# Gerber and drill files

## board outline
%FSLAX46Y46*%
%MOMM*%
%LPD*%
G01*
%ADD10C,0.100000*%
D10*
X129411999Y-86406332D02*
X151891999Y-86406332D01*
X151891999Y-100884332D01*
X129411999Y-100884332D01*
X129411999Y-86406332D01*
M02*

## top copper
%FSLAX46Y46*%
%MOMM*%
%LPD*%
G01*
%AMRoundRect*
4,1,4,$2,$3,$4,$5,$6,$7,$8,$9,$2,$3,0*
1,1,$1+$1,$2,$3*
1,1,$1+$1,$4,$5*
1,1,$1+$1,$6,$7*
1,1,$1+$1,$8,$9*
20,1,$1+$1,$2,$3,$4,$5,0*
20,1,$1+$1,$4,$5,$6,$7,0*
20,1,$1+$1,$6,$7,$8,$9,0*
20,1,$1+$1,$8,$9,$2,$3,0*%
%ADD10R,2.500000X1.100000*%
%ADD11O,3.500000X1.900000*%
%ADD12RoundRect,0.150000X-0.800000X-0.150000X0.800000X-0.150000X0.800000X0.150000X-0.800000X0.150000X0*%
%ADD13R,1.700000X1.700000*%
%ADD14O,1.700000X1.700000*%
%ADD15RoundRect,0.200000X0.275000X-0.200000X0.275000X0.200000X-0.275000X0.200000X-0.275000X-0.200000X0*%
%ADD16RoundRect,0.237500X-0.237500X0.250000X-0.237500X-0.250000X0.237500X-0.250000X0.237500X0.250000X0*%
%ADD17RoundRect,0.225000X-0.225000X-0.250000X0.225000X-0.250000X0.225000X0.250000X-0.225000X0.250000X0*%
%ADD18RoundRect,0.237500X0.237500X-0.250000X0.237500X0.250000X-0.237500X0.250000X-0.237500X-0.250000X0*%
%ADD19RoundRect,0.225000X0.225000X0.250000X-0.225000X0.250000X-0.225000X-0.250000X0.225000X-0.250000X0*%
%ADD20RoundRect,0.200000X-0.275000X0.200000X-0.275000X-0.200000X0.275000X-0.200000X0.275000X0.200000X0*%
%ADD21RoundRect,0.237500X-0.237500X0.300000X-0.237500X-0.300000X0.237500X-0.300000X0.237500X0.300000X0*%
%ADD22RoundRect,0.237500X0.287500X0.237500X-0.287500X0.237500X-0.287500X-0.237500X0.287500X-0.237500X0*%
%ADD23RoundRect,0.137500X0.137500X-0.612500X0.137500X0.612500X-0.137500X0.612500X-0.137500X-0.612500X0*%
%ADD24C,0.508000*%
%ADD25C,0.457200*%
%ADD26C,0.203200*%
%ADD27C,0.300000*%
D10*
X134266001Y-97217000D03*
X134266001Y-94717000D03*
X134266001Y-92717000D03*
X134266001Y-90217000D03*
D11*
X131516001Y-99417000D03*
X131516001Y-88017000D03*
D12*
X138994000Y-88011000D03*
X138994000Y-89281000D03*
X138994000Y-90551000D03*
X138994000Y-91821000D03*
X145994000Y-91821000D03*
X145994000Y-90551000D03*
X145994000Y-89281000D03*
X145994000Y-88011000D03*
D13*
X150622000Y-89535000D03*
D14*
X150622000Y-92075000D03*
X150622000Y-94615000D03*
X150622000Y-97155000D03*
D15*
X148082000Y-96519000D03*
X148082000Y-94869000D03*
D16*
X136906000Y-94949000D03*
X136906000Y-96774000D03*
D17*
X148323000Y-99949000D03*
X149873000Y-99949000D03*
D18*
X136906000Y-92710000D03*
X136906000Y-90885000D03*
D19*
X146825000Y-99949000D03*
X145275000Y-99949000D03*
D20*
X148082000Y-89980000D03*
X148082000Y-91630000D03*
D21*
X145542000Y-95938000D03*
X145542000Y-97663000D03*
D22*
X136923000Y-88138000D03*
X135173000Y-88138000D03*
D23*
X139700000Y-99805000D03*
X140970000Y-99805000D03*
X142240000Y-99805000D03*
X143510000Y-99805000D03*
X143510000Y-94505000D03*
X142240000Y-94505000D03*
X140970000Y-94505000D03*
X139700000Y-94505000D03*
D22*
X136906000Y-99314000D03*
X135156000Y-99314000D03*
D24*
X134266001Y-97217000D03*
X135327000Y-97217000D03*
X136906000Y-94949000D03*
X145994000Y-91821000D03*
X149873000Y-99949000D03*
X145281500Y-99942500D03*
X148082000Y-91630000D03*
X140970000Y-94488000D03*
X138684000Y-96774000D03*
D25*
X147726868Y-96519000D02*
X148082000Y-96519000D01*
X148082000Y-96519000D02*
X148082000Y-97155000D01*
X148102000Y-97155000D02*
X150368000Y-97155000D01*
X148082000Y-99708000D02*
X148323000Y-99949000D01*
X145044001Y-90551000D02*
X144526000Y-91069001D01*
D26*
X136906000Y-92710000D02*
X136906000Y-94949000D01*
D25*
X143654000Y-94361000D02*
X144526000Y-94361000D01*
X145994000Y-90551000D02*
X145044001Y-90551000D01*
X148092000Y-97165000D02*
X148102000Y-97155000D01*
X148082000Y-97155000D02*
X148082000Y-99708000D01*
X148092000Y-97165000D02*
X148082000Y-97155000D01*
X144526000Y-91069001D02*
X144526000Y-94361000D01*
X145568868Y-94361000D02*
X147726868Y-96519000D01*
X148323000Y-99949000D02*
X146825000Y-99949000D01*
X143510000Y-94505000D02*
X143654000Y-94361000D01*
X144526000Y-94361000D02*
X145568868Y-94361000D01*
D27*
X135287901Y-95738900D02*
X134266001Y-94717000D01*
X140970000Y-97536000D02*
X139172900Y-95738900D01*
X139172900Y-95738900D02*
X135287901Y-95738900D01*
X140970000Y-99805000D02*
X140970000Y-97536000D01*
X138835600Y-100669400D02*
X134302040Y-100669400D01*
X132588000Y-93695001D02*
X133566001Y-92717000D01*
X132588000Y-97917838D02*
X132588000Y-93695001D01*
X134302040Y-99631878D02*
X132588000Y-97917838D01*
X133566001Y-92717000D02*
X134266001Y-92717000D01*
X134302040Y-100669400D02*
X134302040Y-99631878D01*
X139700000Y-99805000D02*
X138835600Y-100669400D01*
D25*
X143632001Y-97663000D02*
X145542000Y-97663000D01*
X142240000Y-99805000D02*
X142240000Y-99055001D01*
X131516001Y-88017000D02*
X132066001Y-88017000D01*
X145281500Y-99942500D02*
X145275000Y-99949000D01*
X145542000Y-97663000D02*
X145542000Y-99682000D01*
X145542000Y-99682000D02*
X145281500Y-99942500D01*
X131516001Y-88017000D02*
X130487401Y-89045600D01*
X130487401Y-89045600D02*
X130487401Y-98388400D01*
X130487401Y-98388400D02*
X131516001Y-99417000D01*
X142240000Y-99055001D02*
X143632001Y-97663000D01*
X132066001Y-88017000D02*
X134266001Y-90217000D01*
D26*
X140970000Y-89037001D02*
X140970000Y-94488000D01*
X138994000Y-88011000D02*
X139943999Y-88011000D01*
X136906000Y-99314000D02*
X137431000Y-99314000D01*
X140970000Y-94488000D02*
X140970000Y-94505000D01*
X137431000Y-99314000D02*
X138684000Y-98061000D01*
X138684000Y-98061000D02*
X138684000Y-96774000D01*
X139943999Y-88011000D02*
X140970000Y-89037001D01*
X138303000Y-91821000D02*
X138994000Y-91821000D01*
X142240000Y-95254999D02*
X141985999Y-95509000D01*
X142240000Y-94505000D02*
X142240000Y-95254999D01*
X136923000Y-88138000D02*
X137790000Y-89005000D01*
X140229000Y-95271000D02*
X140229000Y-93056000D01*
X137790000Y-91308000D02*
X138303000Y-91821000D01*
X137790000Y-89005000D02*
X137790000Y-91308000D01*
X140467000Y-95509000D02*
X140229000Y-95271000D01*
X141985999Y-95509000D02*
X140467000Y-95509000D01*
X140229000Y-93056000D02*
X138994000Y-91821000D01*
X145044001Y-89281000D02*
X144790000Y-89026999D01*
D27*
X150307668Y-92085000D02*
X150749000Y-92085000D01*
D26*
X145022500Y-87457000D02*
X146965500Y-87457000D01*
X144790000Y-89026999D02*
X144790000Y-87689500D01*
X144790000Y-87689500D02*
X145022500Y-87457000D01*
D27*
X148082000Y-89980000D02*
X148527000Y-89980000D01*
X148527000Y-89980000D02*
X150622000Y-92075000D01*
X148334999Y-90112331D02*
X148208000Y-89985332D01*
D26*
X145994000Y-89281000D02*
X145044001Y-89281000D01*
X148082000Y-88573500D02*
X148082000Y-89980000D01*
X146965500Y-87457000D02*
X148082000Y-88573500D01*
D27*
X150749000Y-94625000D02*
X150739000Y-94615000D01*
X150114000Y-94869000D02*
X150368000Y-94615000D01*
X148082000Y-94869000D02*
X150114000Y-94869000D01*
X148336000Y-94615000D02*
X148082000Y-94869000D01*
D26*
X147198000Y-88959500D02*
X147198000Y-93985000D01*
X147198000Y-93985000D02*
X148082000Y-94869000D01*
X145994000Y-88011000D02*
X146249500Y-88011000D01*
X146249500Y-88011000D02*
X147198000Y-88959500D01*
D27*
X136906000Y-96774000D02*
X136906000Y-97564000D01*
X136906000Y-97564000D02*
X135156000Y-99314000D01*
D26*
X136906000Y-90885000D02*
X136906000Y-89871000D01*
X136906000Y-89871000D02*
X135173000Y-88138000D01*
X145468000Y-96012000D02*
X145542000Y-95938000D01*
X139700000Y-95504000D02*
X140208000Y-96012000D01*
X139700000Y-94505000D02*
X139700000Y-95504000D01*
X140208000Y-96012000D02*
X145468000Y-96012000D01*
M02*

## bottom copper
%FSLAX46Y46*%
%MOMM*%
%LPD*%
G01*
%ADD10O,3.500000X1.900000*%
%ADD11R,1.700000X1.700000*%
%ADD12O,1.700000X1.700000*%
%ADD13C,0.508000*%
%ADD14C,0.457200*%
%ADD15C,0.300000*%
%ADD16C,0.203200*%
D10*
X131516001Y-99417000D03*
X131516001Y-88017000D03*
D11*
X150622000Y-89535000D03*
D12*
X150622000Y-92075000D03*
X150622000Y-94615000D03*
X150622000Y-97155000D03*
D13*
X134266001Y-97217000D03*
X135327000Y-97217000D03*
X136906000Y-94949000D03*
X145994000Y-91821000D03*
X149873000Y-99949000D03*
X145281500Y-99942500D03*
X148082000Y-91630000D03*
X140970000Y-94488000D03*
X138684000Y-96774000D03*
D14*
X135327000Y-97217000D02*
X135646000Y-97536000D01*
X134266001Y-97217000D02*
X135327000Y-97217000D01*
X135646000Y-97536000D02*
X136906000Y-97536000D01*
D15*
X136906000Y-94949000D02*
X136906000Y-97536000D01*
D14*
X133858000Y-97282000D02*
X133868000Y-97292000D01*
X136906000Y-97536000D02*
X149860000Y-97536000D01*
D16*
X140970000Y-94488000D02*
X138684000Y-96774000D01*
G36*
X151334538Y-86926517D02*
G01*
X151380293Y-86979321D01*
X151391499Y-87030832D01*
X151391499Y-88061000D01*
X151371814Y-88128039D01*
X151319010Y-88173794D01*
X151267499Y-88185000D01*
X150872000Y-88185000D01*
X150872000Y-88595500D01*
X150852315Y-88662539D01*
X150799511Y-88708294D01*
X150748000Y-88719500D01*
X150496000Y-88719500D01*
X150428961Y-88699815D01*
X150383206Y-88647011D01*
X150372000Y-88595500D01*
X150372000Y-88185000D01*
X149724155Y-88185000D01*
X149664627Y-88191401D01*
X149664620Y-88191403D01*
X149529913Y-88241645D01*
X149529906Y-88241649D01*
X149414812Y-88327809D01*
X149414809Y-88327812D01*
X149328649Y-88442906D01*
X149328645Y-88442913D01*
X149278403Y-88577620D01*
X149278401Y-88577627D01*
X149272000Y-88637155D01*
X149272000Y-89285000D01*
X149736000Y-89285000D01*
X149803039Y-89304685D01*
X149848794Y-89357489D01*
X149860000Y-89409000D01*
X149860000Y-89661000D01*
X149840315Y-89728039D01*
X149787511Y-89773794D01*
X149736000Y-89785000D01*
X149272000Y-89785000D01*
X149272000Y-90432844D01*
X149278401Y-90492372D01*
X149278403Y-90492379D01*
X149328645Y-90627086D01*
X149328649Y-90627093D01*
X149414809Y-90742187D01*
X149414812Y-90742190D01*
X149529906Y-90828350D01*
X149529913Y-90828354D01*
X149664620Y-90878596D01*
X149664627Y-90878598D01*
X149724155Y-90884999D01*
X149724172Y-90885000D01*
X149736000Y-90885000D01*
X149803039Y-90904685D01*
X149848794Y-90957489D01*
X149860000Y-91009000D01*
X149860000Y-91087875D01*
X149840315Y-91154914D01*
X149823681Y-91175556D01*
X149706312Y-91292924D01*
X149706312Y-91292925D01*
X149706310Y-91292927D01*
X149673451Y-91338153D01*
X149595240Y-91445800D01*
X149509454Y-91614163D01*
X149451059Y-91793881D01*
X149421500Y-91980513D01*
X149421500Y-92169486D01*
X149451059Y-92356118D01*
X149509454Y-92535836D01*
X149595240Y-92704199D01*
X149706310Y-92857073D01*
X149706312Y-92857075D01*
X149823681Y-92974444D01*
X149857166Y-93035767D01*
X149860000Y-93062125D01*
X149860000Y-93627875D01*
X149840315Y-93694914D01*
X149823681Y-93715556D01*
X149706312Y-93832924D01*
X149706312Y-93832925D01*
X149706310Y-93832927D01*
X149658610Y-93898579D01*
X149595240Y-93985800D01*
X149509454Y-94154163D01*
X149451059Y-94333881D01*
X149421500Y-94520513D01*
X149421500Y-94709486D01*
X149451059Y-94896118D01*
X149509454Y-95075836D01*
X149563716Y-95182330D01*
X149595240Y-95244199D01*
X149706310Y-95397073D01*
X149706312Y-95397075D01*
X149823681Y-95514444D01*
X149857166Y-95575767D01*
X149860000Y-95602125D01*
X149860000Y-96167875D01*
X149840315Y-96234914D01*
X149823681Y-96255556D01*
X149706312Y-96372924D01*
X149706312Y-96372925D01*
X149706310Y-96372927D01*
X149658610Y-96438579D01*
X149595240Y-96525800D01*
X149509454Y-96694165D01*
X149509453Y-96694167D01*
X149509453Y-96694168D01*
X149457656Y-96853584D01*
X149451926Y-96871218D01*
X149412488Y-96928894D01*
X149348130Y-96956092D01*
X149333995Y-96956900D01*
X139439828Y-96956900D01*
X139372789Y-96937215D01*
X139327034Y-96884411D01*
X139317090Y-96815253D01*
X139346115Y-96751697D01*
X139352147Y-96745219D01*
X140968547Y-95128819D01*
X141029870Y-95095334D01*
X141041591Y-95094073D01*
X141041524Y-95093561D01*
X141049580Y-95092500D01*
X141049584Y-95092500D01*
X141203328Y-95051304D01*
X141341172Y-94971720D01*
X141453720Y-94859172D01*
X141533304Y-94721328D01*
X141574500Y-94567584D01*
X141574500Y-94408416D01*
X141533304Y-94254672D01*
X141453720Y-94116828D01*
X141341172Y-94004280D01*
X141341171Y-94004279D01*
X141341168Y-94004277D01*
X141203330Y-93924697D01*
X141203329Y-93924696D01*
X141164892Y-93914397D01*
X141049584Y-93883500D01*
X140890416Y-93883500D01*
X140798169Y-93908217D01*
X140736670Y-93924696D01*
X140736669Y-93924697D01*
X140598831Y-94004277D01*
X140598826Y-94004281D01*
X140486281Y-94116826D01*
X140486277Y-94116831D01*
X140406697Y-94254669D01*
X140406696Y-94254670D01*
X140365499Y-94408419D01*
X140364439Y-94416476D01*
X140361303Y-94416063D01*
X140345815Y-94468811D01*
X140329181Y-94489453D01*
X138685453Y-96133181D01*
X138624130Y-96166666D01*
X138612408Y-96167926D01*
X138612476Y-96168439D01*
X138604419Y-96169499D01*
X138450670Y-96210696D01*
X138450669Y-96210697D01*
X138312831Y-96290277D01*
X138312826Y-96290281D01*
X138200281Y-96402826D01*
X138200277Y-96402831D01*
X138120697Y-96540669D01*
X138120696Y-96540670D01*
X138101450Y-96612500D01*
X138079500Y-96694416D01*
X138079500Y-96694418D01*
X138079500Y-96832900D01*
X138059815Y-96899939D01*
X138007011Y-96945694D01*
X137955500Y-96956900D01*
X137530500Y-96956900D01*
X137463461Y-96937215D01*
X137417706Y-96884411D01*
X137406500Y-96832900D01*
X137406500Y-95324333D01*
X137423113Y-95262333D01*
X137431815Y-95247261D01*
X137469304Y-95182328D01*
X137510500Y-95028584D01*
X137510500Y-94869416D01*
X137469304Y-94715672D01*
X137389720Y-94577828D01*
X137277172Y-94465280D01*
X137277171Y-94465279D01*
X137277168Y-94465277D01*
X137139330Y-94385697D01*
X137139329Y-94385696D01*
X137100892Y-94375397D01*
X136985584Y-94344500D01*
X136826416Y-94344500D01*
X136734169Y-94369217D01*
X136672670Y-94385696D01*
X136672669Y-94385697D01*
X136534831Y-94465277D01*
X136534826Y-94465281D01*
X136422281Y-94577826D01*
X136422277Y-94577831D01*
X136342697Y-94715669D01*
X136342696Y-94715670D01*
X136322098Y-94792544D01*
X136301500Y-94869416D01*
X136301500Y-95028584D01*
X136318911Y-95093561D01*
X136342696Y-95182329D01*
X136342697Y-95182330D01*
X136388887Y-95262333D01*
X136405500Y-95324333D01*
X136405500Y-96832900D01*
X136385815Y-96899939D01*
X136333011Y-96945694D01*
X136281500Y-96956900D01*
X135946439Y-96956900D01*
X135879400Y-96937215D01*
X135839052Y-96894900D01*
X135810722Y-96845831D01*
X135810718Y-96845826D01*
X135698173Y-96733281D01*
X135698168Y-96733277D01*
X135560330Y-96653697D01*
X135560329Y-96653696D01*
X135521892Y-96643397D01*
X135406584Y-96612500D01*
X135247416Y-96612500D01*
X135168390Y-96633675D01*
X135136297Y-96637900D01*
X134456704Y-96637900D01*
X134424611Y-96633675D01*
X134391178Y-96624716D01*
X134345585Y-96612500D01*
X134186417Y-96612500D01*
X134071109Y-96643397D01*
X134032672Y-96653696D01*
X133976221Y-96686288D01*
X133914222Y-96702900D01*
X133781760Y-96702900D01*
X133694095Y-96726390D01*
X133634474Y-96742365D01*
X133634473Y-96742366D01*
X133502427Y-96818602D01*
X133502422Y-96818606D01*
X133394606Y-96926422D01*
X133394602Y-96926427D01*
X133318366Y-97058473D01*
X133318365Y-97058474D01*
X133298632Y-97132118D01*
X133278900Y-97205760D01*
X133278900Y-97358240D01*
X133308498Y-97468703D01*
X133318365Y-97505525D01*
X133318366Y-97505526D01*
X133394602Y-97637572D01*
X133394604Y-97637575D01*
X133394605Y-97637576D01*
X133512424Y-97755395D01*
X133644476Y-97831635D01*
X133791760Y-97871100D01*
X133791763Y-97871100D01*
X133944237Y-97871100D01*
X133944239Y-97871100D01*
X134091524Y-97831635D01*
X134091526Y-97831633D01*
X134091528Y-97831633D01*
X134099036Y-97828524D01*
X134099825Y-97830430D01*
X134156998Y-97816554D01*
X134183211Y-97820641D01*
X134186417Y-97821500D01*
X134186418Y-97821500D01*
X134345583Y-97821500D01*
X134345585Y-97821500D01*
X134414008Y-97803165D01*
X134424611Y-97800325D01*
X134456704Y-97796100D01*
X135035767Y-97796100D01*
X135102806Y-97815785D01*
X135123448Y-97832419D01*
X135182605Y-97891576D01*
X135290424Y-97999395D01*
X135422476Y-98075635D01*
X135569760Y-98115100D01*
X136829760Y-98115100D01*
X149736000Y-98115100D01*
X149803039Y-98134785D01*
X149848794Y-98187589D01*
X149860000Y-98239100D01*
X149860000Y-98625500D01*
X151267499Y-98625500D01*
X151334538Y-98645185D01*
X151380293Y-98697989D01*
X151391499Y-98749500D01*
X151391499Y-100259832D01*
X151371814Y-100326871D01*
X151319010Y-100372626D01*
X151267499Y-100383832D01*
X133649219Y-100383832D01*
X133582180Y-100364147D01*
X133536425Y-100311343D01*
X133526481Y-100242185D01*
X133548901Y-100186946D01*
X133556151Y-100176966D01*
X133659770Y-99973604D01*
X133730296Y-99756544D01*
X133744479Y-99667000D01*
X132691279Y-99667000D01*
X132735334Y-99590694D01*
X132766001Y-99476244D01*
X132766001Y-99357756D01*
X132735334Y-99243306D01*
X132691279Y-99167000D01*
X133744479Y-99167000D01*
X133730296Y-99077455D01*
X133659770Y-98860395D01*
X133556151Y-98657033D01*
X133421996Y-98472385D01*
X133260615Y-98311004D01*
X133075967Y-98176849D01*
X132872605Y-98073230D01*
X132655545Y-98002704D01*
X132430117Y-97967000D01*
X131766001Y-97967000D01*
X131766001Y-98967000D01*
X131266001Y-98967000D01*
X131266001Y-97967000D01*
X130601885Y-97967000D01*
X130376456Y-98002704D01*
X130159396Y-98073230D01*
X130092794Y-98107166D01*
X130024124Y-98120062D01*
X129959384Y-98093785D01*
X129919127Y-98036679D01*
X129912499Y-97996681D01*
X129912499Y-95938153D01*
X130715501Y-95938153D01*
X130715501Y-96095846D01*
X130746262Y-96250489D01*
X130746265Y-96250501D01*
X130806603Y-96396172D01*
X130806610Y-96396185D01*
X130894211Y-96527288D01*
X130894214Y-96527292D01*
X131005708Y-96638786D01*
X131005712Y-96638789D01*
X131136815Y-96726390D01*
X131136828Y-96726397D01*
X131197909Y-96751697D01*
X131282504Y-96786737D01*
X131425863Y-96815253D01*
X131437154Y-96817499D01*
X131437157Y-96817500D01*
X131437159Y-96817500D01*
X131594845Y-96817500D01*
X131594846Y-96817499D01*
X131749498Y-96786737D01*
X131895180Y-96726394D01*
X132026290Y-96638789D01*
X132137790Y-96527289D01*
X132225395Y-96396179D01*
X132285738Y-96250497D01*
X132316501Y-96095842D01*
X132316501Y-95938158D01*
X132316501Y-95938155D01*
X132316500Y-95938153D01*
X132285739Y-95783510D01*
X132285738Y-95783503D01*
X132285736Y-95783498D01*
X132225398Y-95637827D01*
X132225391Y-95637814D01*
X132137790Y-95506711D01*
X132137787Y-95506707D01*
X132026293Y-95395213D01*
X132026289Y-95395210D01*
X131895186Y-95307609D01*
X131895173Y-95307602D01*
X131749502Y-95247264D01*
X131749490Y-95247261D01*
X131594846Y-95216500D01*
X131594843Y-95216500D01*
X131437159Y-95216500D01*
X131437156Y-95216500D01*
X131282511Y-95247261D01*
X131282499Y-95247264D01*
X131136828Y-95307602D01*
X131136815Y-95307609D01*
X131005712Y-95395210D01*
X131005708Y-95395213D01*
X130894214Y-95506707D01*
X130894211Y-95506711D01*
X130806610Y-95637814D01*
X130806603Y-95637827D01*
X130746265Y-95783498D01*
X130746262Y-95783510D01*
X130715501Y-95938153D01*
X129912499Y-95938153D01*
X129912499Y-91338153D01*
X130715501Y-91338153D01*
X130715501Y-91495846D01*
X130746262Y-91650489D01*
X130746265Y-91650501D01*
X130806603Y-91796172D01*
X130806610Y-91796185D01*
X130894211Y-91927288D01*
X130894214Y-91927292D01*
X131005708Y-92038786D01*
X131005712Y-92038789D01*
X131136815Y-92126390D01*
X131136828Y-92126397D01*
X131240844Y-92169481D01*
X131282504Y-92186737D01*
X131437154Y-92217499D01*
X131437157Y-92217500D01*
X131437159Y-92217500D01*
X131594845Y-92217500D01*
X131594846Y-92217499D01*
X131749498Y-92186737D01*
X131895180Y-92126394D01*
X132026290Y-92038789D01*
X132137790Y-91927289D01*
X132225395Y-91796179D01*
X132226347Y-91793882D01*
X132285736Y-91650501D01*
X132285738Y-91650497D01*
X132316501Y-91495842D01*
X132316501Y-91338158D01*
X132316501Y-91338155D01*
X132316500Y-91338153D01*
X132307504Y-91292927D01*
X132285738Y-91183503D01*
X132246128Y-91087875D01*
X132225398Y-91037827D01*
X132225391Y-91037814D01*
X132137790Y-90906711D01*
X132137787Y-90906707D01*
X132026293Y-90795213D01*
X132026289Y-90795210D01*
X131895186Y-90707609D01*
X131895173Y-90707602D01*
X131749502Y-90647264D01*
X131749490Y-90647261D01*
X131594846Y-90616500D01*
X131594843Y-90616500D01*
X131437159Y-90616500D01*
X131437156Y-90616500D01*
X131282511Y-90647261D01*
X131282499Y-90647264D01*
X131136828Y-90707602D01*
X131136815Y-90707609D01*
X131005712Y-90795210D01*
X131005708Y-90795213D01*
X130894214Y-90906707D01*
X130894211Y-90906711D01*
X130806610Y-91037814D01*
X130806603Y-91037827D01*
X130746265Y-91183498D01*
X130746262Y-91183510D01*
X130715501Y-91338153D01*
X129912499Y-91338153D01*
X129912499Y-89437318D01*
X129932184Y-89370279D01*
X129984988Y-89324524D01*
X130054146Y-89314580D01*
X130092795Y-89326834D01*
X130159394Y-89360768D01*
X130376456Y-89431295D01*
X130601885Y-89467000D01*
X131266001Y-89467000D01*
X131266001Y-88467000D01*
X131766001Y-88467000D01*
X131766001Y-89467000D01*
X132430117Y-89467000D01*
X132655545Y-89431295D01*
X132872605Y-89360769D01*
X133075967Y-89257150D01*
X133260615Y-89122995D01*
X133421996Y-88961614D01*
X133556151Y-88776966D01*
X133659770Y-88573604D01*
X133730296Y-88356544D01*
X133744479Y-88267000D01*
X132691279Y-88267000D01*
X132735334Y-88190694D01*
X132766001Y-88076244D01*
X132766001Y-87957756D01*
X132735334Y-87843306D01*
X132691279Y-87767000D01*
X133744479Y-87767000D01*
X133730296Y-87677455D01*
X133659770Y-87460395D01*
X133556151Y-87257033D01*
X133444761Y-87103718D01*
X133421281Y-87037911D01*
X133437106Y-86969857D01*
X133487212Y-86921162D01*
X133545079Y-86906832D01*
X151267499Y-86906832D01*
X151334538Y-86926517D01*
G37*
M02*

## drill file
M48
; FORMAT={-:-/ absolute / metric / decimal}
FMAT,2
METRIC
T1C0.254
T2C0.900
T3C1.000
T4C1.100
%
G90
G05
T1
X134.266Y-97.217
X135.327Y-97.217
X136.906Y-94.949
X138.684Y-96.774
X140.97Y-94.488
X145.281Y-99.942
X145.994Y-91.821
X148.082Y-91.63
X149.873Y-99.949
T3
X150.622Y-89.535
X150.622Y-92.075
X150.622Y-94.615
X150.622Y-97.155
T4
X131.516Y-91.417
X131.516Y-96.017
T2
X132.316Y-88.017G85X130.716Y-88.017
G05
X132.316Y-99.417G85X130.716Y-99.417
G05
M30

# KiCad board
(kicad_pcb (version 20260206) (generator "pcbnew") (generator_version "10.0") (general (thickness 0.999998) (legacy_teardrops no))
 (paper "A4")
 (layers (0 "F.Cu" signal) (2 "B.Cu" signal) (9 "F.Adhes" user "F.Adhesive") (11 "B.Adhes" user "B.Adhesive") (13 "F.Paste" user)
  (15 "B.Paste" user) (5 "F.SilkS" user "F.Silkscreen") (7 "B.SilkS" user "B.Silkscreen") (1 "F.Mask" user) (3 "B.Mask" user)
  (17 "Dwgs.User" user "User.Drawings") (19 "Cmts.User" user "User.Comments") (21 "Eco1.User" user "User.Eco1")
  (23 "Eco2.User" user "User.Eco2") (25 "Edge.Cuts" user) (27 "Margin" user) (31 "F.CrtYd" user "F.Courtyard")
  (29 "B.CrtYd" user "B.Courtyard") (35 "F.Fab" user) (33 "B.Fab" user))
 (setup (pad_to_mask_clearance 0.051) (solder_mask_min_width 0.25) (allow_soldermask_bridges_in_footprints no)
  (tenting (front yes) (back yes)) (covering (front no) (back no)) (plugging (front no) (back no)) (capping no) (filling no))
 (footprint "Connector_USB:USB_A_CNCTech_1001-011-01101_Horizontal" (layer "F.Cu") (at 124.616001 93.717 180)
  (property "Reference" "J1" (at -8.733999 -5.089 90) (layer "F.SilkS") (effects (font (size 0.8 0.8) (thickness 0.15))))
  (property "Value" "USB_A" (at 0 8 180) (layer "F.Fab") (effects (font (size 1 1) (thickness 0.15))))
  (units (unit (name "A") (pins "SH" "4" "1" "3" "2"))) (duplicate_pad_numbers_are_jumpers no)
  (pad "" np_thru_hole circle (at -6.9 -2.3 180) (size 1.1 1.1) (drill 1.1) (layers "*.Cu" "*.Mask"))
  (pad "" np_thru_hole circle (at -6.9 2.3 180) (size 1.1 1.1) (drill 1.1) (layers "*.Cu" "*.Mask"))
  (pad "1" smd rect (at -9.65 -3.5 180) (size 2.5 1.1) (layers "F.Cu" "F.Mask" "F.Paste") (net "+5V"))
  (pad "2" smd rect (at -9.65 -1 180) (size 2.5 1.1) (layers "F.Cu" "F.Mask" "F.Paste") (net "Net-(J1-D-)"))
  (pad "3" smd rect (at -9.65 1 180) (size 2.5 1.1) (layers "F.Cu" "F.Mask" "F.Paste") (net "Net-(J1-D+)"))
  (pad "4" smd rect (at -9.65 3.5 180) (size 2.5 1.1) (layers "F.Cu" "F.Mask" "F.Paste") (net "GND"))
  (pad "SH" thru_hole oval (at -6.9 -5.7 180) (size 3.5 1.9) (drill oval 2.5 0.9) (layers "*.Cu" "*.Mask") (remove_unused_layers no)
   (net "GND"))
  (pad "SH" thru_hole oval (at -6.9 5.7 180) (size 3.5 1.9) (drill oval 2.5 0.9) (layers "*.Cu" "*.Mask") (remove_unused_layers no)
   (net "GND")))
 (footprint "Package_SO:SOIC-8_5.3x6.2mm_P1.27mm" (layer "F.Cu") (at 142.494 89.916)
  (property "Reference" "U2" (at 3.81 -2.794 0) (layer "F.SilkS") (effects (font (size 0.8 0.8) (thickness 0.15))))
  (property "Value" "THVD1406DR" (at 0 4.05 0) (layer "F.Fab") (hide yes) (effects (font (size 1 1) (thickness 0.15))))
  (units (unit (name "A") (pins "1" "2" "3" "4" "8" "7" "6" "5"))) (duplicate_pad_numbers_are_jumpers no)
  (pad "1" smd roundrect (at -3.5 -1.905) (size 1.9 0.6) (layers "F.Cu" "F.Mask" "F.Paste") (roundrect_rratio 0.25) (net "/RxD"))
  (pad "2" smd roundrect (at -3.5 -0.635) (size 1.9 0.6) (layers "F.Cu" "F.Mask" "F.Paste") (roundrect_rratio 0.25)
   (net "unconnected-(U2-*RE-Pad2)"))
  (pad "3" smd roundrect (at -3.5 0.635) (size 1.9 0.6) (layers "F.Cu" "F.Mask" "F.Paste") (roundrect_rratio 0.25)
   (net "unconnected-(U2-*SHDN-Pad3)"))
  (pad "4" smd roundrect (at -3.5 1.905) (size 1.9 0.6) (layers "F.Cu" "F.Mask" "F.Paste") (roundrect_rratio 0.25) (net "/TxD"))
  (pad "5" smd roundrect (at 3.5 1.905) (size 1.9 0.6) (layers "F.Cu" "F.Mask" "F.Paste") (roundrect_rratio 0.25) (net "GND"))
  (pad "6" smd roundrect (at 3.5 0.635) (size 1.9 0.6) (layers "F.Cu" "F.Mask" "F.Paste") (roundrect_rratio 0.25) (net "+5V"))
  (pad "7" smd roundrect (at 3.5 -0.635) (size 1.9 0.6) (layers "F.Cu" "F.Mask" "F.Paste") (roundrect_rratio 0.25) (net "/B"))
  (pad "8" smd roundrect (at 3.5 -1.905) (size 1.9 0.6) (layers "F.Cu" "F.Mask" "F.Paste") (roundrect_rratio 0.25) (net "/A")))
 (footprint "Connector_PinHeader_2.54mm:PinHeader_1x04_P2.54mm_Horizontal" (layer "F.Cu") (at 150.622 89.535)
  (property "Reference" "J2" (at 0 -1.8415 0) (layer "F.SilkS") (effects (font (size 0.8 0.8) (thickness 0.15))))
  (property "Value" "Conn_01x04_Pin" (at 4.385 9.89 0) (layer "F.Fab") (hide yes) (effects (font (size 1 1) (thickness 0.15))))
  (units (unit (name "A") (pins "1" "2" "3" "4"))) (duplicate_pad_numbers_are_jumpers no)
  (pad "1" thru_hole rect (at 0 0) (size 1.7 1.7) (drill 1) (layers "*.Cu" "*.Mask") (remove_unused_layers no) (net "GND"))
  (pad "2" thru_hole oval (at 0 2.54) (size 1.7 1.7) (drill 1) (layers "*.Cu" "*.Mask") (remove_unused_layers no) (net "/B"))
  (pad "3" thru_hole oval (at 0 5.08) (size 1.7 1.7) (drill 1) (layers "*.Cu" "*.Mask") (remove_unused_layers no) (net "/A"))
  (pad "4" thru_hole oval (at 0 7.62) (size 1.7 1.7) (drill 1) (layers "*.Cu" "*.Mask") (remove_unused_layers no) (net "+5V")))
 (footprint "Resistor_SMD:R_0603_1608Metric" (layer "F.Cu") (at 148.082 95.694 90)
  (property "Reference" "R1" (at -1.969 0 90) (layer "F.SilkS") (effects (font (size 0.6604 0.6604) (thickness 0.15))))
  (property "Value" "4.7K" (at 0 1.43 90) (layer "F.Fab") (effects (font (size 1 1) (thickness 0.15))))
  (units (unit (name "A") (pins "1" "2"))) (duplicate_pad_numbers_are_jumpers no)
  (pad "1" smd roundrect (at -0.825 0 90) (size 0.8 0.95) (layers "F.Cu" "F.Mask" "F.Paste") (roundrect_rratio 0.25) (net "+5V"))
  (pad "2" smd roundrect (at 0.825 0 90) (size 0.8 0.95) (layers "F.Cu" "F.Mask" "F.Paste") (roundrect_rratio 0.25) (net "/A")))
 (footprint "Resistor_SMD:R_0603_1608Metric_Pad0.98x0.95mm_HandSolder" (layer "F.Cu") (at 136.906 95.8615 -90)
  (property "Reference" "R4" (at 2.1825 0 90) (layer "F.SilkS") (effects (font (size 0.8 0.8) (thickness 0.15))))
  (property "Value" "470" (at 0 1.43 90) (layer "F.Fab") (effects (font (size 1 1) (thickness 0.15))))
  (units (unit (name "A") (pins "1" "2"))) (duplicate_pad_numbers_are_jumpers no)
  (pad "1" smd roundrect (at -0.9125 0 270) (size 0.975 0.95) (layers "F.Cu" "F.Mask" "F.Paste") (roundrect_rratio 0.25) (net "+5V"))
  (pad "2" smd roundrect (at 0.9125 0 270) (size 0.975 0.95) (layers "F.Cu" "F.Mask" "F.Paste") (roundrect_rratio 0.25) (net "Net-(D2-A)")))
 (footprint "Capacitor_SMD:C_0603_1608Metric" (layer "F.Cu") (at 149.098 99.949)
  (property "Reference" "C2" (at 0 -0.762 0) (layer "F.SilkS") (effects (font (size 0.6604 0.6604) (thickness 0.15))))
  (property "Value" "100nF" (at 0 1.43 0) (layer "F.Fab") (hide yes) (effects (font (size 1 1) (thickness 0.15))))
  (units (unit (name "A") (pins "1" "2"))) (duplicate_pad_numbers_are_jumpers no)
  (pad "1" smd roundrect (at -0.775 0) (size 0.9 0.95) (layers "F.Cu" "F.Mask" "F.Paste") (roundrect_rratio 0.25) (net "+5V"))
  (pad "2" smd roundrect (at 0.775 0) (size 0.9 0.95) (layers "F.Cu" "F.Mask" "F.Paste") (roundrect_rratio 0.25) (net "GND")))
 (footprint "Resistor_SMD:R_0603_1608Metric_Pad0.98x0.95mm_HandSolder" (layer "F.Cu") (at 136.906 91.7975 90)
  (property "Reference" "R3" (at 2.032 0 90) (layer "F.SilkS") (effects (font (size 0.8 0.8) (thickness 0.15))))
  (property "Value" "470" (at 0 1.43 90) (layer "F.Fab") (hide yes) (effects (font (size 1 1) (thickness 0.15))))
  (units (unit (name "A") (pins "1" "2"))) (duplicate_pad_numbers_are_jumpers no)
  (pad "1" smd roundrect (at -0.9125 0 90) (size 0.975 0.95) (layers "F.Cu" "F.Mask" "F.Paste") (roundrect_rratio 0.25) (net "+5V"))
  (pad "2" smd roundrect (at 0.9125 0 90) (size 0.975 0.95) (layers "F.Cu" "F.Mask" "F.Paste") (roundrect_rratio 0.25) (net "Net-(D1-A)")))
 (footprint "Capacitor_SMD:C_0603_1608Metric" (layer "F.Cu") (at 146.05 99.949 180)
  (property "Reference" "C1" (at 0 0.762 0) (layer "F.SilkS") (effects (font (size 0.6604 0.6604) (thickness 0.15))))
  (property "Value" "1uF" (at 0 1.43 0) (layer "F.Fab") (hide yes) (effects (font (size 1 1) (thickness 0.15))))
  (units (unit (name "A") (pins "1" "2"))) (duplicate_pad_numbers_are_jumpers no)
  (pad "1" smd roundrect (at -0.775 0 180) (size 0.9 0.95) (layers "F.Cu" "F.Mask" "F.Paste") (roundrect_rratio 0.25) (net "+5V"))
  (pad "2" smd roundrect (at 0.775 0 180) (size 0.9 0.95) (layers "F.Cu" "F.Mask" "F.Paste") (roundrect_rratio 0.25) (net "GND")))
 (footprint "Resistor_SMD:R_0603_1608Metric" (layer "F.Cu") (at 148.082 90.805 -90)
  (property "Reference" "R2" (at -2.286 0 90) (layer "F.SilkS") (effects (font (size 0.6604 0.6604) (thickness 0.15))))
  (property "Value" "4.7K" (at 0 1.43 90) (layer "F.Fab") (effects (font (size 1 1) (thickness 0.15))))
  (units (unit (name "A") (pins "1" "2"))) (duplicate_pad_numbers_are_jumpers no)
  (pad "1" smd roundrect (at -0.825 0 270) (size 0.8 0.95) (layers "F.Cu" "F.Mask" "F.Paste") (roundrect_rratio 0.25) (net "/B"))
  (pad "2" smd roundrect (at 0.825 0 270) (size 0.8 0.95) (layers "F.Cu" "F.Mask" "F.Paste") (roundrect_rratio 0.25) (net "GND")))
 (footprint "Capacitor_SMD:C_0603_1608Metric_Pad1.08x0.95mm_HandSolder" (layer "F.Cu") (at 145.542 96.8005 -90)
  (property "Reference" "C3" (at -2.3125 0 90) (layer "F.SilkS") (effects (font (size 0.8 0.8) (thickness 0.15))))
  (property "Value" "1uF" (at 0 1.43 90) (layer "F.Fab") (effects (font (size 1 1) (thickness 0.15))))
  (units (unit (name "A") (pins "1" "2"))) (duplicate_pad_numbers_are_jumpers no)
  (pad "1" smd roundrect (at -0.8625 0 270) (size 1.075 0.95) (layers "F.Cu" "F.Mask" "F.Paste") (roundrect_rratio 0.25) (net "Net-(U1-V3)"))
  (pad "2" smd roundrect (at 0.8625 0 270) (size 1.075 0.95) (layers "F.Cu" "F.Mask" "F.Paste") (roundrect_rratio 0.25) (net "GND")))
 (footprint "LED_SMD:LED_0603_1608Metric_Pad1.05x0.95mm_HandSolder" (layer "F.Cu") (at 136.048 88.138 180)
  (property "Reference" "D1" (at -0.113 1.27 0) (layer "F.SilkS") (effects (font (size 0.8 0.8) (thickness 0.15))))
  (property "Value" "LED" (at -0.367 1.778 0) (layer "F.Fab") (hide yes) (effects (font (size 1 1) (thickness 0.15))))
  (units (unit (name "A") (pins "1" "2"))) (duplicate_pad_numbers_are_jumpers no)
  (pad "1" smd roundrect (at -0.875 0 180) (size 1.05 0.95) (layers "F.Cu" "F.Mask" "F.Paste") (roundrect_rratio 0.25) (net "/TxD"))
  (pad "2" smd roundrect (at 0.875 0 180) (size 1.05 0.95) (layers "F.Cu" "F.Mask" "F.Paste") (roundrect_rratio 0.25) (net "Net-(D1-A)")))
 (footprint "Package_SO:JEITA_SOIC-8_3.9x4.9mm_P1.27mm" (layer "F.Cu") (at 141.605 97.155 90)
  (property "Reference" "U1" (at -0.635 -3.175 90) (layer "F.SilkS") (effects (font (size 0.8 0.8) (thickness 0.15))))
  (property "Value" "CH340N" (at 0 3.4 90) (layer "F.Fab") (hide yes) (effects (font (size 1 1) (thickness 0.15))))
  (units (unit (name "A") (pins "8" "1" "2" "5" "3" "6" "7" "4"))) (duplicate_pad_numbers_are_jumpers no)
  (pad "1" smd roundrect (at -2.65 -1.905 90) (size 1.5 0.55) (layers "F.Cu" "F.Mask" "F.Paste") (roundrect_rratio 0.25) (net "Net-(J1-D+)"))
  (pad "2" smd roundrect (at -2.65 -0.635 90) (size 1.5 0.55) (layers "F.Cu" "F.Mask" "F.Paste") (roundrect_rratio 0.25) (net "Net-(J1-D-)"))
  (pad "3" smd roundrect (at -2.65 0.635 90) (size 1.5 0.55) (layers "F.Cu" "F.Mask" "F.Paste") (roundrect_rratio 0.25) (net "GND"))
  (pad "4" smd roundrect (at -2.65 1.905 90) (size 1.5 0.55) (layers "F.Cu" "F.Mask" "F.Paste") (roundrect_rratio 0.25)
   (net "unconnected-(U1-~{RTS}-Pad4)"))
  (pad "5" smd roundrect (at 2.65 1.905 90) (size 1.5 0.55) (layers "F.Cu" "F.Mask" "F.Paste") (roundrect_rratio 0.25) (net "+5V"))
  (pad "6" smd roundrect (at 2.65 0.635 90) (size 1.5 0.55) (layers "F.Cu" "F.Mask" "F.Paste") (roundrect_rratio 0.25) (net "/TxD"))
  (pad "7" smd roundrect (at 2.65 -0.635 90) (size 1.5 0.55) (layers "F.Cu" "F.Mask" "F.Paste") (roundrect_rratio 0.25) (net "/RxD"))
  (pad "8" smd roundrect (at 2.65 -1.905 90) (size 1.5 0.55) (layers "F.Cu" "F.Mask" "F.Paste") (roundrect_rratio 0.25) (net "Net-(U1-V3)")))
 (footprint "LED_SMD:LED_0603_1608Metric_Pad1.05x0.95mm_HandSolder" (layer "F.Cu") (at 136.031 99.314 180)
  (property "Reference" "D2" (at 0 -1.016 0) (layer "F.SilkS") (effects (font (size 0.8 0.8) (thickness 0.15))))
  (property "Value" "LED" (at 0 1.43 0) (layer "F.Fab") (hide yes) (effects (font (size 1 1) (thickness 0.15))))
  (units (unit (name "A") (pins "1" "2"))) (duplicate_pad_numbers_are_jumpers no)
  (pad "1" smd roundrect (at -0.875 0 180) (size 1.05 0.95) (layers "F.Cu" "F.Mask" "F.Paste") (roundrect_rratio 0.25) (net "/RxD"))
  (pad "2" smd roundrect (at 0.875 0 180) (size 1.05 0.95) (layers "F.Cu" "F.Mask" "F.Paste") (roundrect_rratio 0.25) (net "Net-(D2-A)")))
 (gr_rect (start 129.411999 86.406332) (end 151.891999 100.884332) (stroke (width 0.1) (type solid)) (fill no) (layer "Edge.Cuts"))
 (segment (start 147.726868 96.519) (end 148.082 96.519) (width 0.4572) (layer "F.Cu") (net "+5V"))
 (segment (start 148.082 96.519) (end 148.082 97.155) (width 0.4572) (layer "F.Cu") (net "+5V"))
 (segment (start 148.102 97.155) (end 150.368 97.155) (width 0.4572) (layer "F.Cu") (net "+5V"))
 (segment (start 148.082 99.708) (end 148.323 99.949) (width 0.4572) (layer "F.Cu") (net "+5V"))
 (segment (start 145.044001 90.551) (end 144.526 91.069001) (width 0.4572) (layer "F.Cu") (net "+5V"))
 (segment (start 136.906 92.71) (end 136.906 94.949) (width 0.2032) (layer "F.Cu") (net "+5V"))
 (segment (start 143.654 94.361) (end 144.526 94.361) (width 0.4572) (layer "F.Cu") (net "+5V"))
 (segment (start 145.994 90.551) (end 145.044001 90.551) (width 0.4572) (layer "F.Cu") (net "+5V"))
 (segment (start 148.092 97.165) (end 148.102 97.155) (width 0.4572) (layer "F.Cu") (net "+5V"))
 (segment (start 148.082 97.155) (end 148.082 99.708) (width 0.4572) (layer "F.Cu") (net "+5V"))
 (segment (start 148.092 97.165) (end 148.082 97.155) (width 0.4572) (layer "F.Cu") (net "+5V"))
 (segment (start 144.526 91.069001) (end 144.526 94.361) (width 0.4572) (layer "F.Cu") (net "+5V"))
 (segment (start 145.568868 94.361) (end 147.726868 96.519) (width 0.4572) (layer "F.Cu") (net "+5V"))
 (segment (start 148.323 99.949) (end 146.825 99.949) (width 0.4572) (layer "F.Cu") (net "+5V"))
 (segment (start 143.51 94.505) (end 143.654 94.361) (width 0.4572) (layer "F.Cu") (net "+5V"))
 (segment (start 144.526 94.361) (end 145.568868 94.361) (width 0.4572) (layer "F.Cu") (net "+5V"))
 (via (at 134.266001 97.217) (size 0.508) (drill 0.254) (layers "F.Cu" "B.Cu") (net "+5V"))
 (via (at 135.327 97.217) (size 0.508) (drill 0.254) (layers "F.Cu" "B.Cu") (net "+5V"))
 (via (at 136.906 94.949) (size 0.508) (drill 0.254) (layers "F.Cu" "B.Cu") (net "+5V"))
 (segment (start 135.327 97.217) (end 135.646 97.536) (width 0.4572) (layer "B.Cu") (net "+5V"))
 (segment (start 134.266001 97.217) (end 135.327 97.217) (width 0.4572) (layer "B.Cu") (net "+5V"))
 (segment (start 135.646 97.536) (end 136.906 97.536) (width 0.4572) (layer "B.Cu") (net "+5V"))
 (segment (start 136.906 94.949) (end 136.906 97.536) (width 0.3) (layer "B.Cu") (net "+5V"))
 (segment (start 133.858 97.282) (end 133.868 97.292) (width 0.4572) (layer "B.Cu") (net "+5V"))
 (segment (start 136.906 97.536) (end 149.86 97.536) (width 0.4572) (layer "B.Cu") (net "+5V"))
 (segment (start 135.287901 95.7389) (end 134.266001 94.717) (width 0.3) (layer "F.Cu") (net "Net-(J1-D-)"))
 (segment (start 140.97 97.536) (end 139.1729 95.7389) (width 0.3) (layer "F.Cu") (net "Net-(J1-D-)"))
 (segment (start 139.1729 95.7389) (end 135.287901 95.7389) (width 0.3) (layer "F.Cu") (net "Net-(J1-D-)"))
 (segment (start 140.97 99.805) (end 140.97 97.536) (width 0.3) (layer "F.Cu") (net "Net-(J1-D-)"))
 (segment (start 138.8356 100.6694) (end 134.30204 100.6694) (width 0.3) (layer "F.Cu") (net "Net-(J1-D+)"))
 (segment (start 132.588 93.695001) (end 133.566001 92.717) (width 0.3) (layer "F.Cu") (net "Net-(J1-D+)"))
 (segment (start 132.588 97.917838) (end 132.588 93.695001) (width 0.3) (layer "F.Cu") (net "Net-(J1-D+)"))
 (segment (start 134.30204 99.631878) (end 132.588 97.917838) (width 0.3) (layer "F.Cu") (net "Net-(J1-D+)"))
 (segment (start 133.566001 92.717) (end 134.266001 92.717) (width 0.3) (layer "F.Cu") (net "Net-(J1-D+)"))
 (segment (start 134.30204 100.6694) (end 134.30204 99.631878) (width 0.3) (layer "F.Cu") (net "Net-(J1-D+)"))
 (segment (start 139.7 99.805) (end 138.8356 100.6694) (width 0.3) (layer "F.Cu") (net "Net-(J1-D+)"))
 (segment (start 143.632001 97.663) (end 145.542 97.663) (width 0.4572) (layer "F.Cu") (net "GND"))
 (segment (start 142.24 99.805) (end 142.24 99.055001) (width 0.4572) (layer "F.Cu") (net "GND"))
 (segment (start 131.516001 88.017) (end 132.066001 88.017) (width 0.4572) (layer "F.Cu") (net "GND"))
 (segment (start 145.2815 99.9425) (end 145.275 99.949) (width 0.4572) (layer "F.Cu") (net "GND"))
 (segment (start 145.542 97.663) (end 145.542 99.682) (width 0.4572) (layer "F.Cu") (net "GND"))
 (segment (start 145.542 99.682) (end 145.2815 99.9425) (width 0.4572) (layer "F.Cu") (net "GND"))
 (segment (start 131.516001 88.017) (end 130.487401 89.0456) (width 0.4572) (layer "F.Cu") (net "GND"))
 (segment (start 130.487401 89.0456) (end 130.487401 98.3884) (width 0.4572) (layer "F.Cu") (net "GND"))
 (segment (start 130.487401 98.3884) (end 131.516001 99.417) (width 0.4572) (layer "F.Cu") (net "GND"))
 (segment (start 142.24 99.055001) (end 143.632001 97.663) (width 0.4572) (layer "F.Cu") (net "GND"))
 (segment (start 132.066001 88.017) (end 134.266001 90.217) (width 0.4572) (layer "F.Cu") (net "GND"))
 (via (at 145.994 91.821) (size 0.508) (drill 0.254) (layers "F.Cu" "B.Cu") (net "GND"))
 (via (at 149.873 99.949) (size 0.508) (drill 0.254) (layers "F.Cu" "B.Cu") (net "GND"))
 (via (at 145.2815 99.9425) (size 0.508) (drill 0.254) (layers "F.Cu" "B.Cu") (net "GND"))
 (via (at 148.082 91.63) (size 0.508) (drill 0.254) (layers "F.Cu" "B.Cu") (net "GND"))
 (segment (start 140.97 89.037001) (end 140.97 94.488) (width 0.2032) (layer "F.Cu") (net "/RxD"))
 (segment (start 138.994 88.011) (end 139.943999 88.011) (width 0.2032) (layer "F.Cu") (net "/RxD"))
 (segment (start 136.906 99.314) (end 137.431 99.314) (width 0.2032) (layer "F.Cu") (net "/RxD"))
 (segment (start 140.97 94.488) (end 140.97 94.505) (width 0.2032) (layer "F.Cu") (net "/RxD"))
 (segment (start 137.431 99.314) (end 138.684 98.061) (width 0.2032) (layer "F.Cu") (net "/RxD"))
 (segment (start 138.684 98.061) (end 138.684 96.774) (width 0.2032) (layer "F.Cu") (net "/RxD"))
 (segment (start 139.943999 88.011) (end 140.97 89.037001) (width 0.2032) (layer "F.Cu") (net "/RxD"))
 (via (at 140.97 94.488) (size 0.508) (drill 0.254) (layers "F.Cu" "B.Cu") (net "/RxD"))
 (via (at 138.684 96.774) (size 0.508) (drill 0.254) (layers "F.Cu" "B.Cu") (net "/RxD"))
 (segment (start 140.97 94.488) (end 138.684 96.774) (width 0.2032) (layer "B.Cu") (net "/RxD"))
 (segment (start 138.303 91.821) (end 138.994 91.821) (width 0.2032) (layer "F.Cu") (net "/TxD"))
 (segment (start 142.24 95.254999) (end 141.985999 95.509) (width 0.2032) (layer "F.Cu") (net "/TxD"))
 (segment (start 142.24 94.505) (end 142.24 95.254999) (width 0.2032) (layer "F.Cu") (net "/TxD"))
 (segment (start 136.923 88.138) (end 137.79 89.005) (width 0.2032) (layer "F.Cu") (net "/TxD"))
 (segment (start 140.229 95.271) (end 140.229 93.056) (width 0.2032) (layer "F.Cu") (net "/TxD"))
 (segment (start 137.79 91.308) (end 138.303 91.821) (width 0.2032) (layer "F.Cu") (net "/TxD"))
 (segment (start 137.79 89.005) (end 137.79 91.308) (width 0.2032) (layer "F.Cu") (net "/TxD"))
 (segment (start 140.467 95.509) (end 140.229 95.271) (width 0.2032) (layer "F.Cu") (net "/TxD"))
 (segment (start 141.985999 95.509) (end 140.467 95.509) (width 0.2032) (layer "F.Cu") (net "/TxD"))
 (segment (start 140.229 93.056) (end 138.994 91.821) (width 0.2032) (layer "F.Cu") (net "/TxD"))
 (segment (start 145.044001 89.281) (end 144.79 89.026999) (width 0.2032) (layer "F.Cu") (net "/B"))
 (segment (start 150.307668 92.085) (end 150.749 92.085) (width 0.3) (layer "F.Cu") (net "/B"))
 (segment (start 145.0225 87.457) (end 146.9655 87.457) (width 0.2032) (layer "F.Cu") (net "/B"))
 (segment (start 144.79 89.026999) (end 144.79 87.6895) (width 0.2032) (layer "F.Cu") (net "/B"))
 (segment (start 144.79 87.6895) (end 145.0225 87.457) (width 0.2032) (layer "F.Cu") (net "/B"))
 (segment (start 148.082 89.98) (end 148.527 89.98) (width 0.3) (layer "F.Cu") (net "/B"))
 (segment (start 148.527 89.98) (end 150.622 92.075) (width 0.3) (layer "F.Cu") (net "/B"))
 (segment (start 148.334999 90.112331) (end 148.208 89.985332) (width 0.3) (layer "F.Cu") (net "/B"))
 (segment (start 145.994 89.281) (end 145.044001 89.281) (width 0.2032) (layer "F.Cu") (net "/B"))
 (segment (start 148.082 88.5735) (end 148.082 89.98) (width 0.2032) (layer "F.Cu") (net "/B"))
 (segment (start 146.9655 87.457) (end 148.082 88.5735) (width 0.2032) (layer "F.Cu") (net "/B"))
 (segment (start 150.749 94.625) (end 150.739 94.615) (width 0.3) (layer "F.Cu") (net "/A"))
 (segment (start 150.114 94.869) (end 150.368 94.615) (width 0.3) (layer "F.Cu") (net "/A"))
 (segment (start 148.082 94.869) (end 150.114 94.869) (width 0.3) (layer "F.Cu") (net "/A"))
 (segment (start 148.336 94.615) (end 148.082 94.869) (width 0.3) (layer "F.Cu") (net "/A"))
 (segment (start 147.198 88.9595) (end 147.198 93.985) (width 0.2032) (layer "F.Cu") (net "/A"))
 (segment (start 147.198 93.985) (end 148.082 94.869) (width 0.2032) (layer "F.Cu") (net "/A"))
 (segment (start 145.994 88.011) (end 146.2495 88.011) (width 0.2032) (layer "F.Cu") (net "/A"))
 (segment (start 146.2495 88.011) (end 147.198 88.9595) (width 0.2032) (layer "F.Cu") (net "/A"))
 (segment (start 136.906 96.774) (end 136.906 97.564) (width 0.3) (layer "F.Cu") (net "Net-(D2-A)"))
 (segment (start 136.906 97.564) (end 135.156 99.314) (width 0.3) (layer "F.Cu") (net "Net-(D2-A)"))
 (segment (start 136.906 90.885) (end 136.906 89.871) (width 0.2032) (layer "F.Cu") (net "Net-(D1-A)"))
 (segment (start 136.906 89.871) (end 135.173 88.138) (width 0.2032) (layer "F.Cu") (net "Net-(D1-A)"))
 (segment (start 145.468 96.012) (end 145.542 95.938) (width 0.2032) (layer "F.Cu") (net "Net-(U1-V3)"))
 (segment (start 139.7 95.504) (end 140.208 96.012) (width 0.2032) (layer "F.Cu") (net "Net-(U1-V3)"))
 (segment (start 139.7 94.505) (end 139.7 95.504) (width 0.2032) (layer "F.Cu") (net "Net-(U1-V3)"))
 (segment (start 140.208 96.012) (end 145.468 96.012) (width 0.2032) (layer "F.Cu") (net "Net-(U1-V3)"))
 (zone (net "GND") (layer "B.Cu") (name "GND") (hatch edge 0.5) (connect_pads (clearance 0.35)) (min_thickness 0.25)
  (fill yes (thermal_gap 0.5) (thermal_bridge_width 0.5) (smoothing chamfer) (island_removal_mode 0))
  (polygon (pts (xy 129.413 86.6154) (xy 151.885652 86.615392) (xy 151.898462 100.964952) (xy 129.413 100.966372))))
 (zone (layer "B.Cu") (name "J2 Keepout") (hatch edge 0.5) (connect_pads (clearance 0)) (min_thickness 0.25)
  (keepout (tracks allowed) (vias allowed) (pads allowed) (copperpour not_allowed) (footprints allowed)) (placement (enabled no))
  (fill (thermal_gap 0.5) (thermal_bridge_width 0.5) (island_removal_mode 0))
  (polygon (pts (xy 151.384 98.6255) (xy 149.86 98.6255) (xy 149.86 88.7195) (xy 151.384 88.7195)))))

